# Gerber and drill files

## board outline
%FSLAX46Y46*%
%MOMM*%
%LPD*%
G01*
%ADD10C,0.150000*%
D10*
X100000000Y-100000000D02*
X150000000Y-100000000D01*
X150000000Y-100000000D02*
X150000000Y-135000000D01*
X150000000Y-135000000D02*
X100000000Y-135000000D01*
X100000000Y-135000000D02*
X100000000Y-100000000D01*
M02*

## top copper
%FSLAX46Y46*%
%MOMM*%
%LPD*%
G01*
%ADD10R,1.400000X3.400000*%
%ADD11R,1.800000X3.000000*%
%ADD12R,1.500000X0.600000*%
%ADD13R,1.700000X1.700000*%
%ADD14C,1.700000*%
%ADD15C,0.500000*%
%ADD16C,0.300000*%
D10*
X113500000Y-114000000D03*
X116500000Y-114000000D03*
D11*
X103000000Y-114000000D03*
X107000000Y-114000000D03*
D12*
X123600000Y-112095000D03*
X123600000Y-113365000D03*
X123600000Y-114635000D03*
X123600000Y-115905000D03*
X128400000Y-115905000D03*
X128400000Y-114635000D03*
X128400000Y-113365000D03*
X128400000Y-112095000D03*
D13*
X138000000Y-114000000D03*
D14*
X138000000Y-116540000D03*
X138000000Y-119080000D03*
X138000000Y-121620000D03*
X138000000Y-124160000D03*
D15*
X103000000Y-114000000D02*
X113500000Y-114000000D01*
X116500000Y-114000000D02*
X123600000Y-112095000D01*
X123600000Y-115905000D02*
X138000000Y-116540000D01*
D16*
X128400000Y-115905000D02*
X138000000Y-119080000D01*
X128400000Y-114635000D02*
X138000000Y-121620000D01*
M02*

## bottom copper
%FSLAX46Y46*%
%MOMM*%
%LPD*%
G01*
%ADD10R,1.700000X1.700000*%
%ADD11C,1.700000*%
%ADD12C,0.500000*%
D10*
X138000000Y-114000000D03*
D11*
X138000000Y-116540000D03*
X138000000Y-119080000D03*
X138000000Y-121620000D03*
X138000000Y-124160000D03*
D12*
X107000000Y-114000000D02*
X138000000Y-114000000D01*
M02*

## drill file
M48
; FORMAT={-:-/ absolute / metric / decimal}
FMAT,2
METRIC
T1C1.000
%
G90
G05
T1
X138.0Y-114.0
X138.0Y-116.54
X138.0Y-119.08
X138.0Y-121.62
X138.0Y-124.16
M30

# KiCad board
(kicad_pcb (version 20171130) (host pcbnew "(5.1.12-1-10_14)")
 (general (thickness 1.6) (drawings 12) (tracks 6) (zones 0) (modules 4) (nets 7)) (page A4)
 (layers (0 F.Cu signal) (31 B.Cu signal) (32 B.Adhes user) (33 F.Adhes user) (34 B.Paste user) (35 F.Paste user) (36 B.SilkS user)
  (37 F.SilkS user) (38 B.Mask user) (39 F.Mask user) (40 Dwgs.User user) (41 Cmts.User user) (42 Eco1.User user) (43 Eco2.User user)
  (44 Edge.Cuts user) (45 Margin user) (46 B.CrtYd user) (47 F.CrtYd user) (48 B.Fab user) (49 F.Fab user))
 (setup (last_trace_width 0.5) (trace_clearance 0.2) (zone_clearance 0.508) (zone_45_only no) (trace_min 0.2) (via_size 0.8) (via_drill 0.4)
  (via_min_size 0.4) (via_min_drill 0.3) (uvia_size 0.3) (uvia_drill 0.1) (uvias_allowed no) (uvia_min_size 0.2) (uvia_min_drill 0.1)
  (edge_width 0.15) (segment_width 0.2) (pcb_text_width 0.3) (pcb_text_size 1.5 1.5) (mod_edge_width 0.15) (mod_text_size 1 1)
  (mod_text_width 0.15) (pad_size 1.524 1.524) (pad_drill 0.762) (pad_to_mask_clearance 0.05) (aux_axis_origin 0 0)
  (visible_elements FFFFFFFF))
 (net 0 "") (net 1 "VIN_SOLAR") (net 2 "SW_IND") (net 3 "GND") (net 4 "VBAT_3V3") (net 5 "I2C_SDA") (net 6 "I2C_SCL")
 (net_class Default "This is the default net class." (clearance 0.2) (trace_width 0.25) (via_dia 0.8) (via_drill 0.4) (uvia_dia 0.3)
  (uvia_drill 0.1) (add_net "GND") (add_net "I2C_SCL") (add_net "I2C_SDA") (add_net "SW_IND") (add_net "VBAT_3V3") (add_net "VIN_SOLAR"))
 (gr_line (start 100 100) (end 150 100) (layer Edge.Cuts) (width 0.15))
 (gr_line (start 150 100) (end 150 135) (layer Edge.Cuts) (width 0.15))
 (gr_line (start 150 135) (end 100 135) (layer Edge.Cuts) (width 0.15))
 (gr_line (start 100 135) (end 100 100) (layer Edge.Cuts) (width 0.15))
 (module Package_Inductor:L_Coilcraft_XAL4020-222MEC (layer F.Cu) (at 115 114)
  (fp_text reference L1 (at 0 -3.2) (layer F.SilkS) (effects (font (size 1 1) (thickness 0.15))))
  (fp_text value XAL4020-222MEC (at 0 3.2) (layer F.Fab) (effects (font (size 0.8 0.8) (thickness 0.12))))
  (pad 1 smd rect (at -1.5 0) (size 1.4 3.4) (layers F.Cu F.Paste F.Mask) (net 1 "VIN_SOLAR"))
  (pad 2 smd rect (at 1.5 0) (size 1.4 3.4) (layers F.Cu F.Paste F.Mask) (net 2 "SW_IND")))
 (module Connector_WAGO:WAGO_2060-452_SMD (layer F.Cu) (at 105 114)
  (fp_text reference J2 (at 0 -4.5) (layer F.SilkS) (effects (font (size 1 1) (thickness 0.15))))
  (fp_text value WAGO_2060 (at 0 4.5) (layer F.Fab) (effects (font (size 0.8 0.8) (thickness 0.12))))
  (pad 1 smd rect (at -2.0 0) (size 1.8 3.0) (layers F.Cu F.Paste F.Mask) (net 1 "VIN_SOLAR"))
  (pad 2 smd rect (at 2.0 0) (size 1.8 3.0) (layers F.Cu F.Paste F.Mask) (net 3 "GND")))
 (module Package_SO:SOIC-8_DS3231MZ (layer F.Cu) (at 126 114)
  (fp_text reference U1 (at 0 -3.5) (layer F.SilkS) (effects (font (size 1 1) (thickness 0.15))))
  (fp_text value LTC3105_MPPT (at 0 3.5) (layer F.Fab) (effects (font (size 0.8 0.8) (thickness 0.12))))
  (pad 1 smd rect (at -2.4 -1.905) (size 1.5 0.6) (layers F.Cu F.Paste F.Mask) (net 2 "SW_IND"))
  (pad 2 smd rect (at -2.4 -0.635) (size 1.5 0.6) (layers F.Cu F.Paste F.Mask) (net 1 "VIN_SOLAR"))
  (pad 3 smd rect (at -2.4 0.635) (size 1.5 0.6) (layers F.Cu F.Paste F.Mask) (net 3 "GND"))
  (pad 4 smd rect (at -2.4 1.905) (size 1.5 0.6) (layers F.Cu F.Paste F.Mask) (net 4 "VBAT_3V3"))
  (pad 5 smd rect (at 2.4 1.905) (size 1.5 0.6) (layers F.Cu F.Paste F.Mask) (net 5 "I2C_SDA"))
  (pad 6 smd rect (at 2.4 0.635) (size 1.5 0.6) (layers F.Cu F.Paste F.Mask) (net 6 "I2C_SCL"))
  (pad 7 smd rect (at 2.4 -0.635) (size 1.5 0.6) (layers F.Cu F.Paste F.Mask) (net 4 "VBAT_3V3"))
  (pad 8 smd rect (at 2.4 -1.905) (size 1.5 0.6) (layers F.Cu F.Paste F.Mask) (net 3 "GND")))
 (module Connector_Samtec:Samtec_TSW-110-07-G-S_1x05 (layer F.Cu) (at 138 114)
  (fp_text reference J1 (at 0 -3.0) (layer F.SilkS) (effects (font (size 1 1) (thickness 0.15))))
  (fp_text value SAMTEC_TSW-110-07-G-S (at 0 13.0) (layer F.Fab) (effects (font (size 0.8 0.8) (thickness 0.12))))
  (pad 1 thru_hole rect (at 0 0) (size 1.7 1.7) (drill 1.0) (layers *.Cu *.Mask) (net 3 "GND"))
  (pad 2 thru_hole circle (at 0 2.54) (size 1.7 1.7) (drill 1.0) (layers *.Cu *.Mask) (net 4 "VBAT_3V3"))
  (pad 3 thru_hole circle (at 0 5.08) (size 1.7 1.7) (drill 1.0) (layers *.Cu *.Mask) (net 5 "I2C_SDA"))
  (pad 4 thru_hole circle (at 0 7.62) (size 1.7 1.7) (drill 1.0) (layers *.Cu *.Mask) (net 6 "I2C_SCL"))
  (pad 5 thru_hole circle (at 0 10.16) (size 1.7 1.7) (drill 1.0) (layers *.Cu *.Mask) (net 1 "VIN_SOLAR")))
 (segment (start 103 114) (end 113.5 114) (width 0.5) (layer F.Cu) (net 1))
 (segment (start 116.5 114) (end 123.6 112.095) (width 0.5) (layer F.Cu) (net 2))
 (segment (start 123.6 115.905) (end 138 116.54) (width 0.5) (layer F.Cu) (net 4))
 (segment (start 128.4 115.905) (end 138 119.08) (width 0.3) (layer F.Cu) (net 5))
 (segment (start 128.4 114.635) (end 138 121.62) (width 0.3) (layer F.Cu) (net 6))
 (segment (start 107 114) (end 138 114) (width 0.5) (layer B.Cu) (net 3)))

